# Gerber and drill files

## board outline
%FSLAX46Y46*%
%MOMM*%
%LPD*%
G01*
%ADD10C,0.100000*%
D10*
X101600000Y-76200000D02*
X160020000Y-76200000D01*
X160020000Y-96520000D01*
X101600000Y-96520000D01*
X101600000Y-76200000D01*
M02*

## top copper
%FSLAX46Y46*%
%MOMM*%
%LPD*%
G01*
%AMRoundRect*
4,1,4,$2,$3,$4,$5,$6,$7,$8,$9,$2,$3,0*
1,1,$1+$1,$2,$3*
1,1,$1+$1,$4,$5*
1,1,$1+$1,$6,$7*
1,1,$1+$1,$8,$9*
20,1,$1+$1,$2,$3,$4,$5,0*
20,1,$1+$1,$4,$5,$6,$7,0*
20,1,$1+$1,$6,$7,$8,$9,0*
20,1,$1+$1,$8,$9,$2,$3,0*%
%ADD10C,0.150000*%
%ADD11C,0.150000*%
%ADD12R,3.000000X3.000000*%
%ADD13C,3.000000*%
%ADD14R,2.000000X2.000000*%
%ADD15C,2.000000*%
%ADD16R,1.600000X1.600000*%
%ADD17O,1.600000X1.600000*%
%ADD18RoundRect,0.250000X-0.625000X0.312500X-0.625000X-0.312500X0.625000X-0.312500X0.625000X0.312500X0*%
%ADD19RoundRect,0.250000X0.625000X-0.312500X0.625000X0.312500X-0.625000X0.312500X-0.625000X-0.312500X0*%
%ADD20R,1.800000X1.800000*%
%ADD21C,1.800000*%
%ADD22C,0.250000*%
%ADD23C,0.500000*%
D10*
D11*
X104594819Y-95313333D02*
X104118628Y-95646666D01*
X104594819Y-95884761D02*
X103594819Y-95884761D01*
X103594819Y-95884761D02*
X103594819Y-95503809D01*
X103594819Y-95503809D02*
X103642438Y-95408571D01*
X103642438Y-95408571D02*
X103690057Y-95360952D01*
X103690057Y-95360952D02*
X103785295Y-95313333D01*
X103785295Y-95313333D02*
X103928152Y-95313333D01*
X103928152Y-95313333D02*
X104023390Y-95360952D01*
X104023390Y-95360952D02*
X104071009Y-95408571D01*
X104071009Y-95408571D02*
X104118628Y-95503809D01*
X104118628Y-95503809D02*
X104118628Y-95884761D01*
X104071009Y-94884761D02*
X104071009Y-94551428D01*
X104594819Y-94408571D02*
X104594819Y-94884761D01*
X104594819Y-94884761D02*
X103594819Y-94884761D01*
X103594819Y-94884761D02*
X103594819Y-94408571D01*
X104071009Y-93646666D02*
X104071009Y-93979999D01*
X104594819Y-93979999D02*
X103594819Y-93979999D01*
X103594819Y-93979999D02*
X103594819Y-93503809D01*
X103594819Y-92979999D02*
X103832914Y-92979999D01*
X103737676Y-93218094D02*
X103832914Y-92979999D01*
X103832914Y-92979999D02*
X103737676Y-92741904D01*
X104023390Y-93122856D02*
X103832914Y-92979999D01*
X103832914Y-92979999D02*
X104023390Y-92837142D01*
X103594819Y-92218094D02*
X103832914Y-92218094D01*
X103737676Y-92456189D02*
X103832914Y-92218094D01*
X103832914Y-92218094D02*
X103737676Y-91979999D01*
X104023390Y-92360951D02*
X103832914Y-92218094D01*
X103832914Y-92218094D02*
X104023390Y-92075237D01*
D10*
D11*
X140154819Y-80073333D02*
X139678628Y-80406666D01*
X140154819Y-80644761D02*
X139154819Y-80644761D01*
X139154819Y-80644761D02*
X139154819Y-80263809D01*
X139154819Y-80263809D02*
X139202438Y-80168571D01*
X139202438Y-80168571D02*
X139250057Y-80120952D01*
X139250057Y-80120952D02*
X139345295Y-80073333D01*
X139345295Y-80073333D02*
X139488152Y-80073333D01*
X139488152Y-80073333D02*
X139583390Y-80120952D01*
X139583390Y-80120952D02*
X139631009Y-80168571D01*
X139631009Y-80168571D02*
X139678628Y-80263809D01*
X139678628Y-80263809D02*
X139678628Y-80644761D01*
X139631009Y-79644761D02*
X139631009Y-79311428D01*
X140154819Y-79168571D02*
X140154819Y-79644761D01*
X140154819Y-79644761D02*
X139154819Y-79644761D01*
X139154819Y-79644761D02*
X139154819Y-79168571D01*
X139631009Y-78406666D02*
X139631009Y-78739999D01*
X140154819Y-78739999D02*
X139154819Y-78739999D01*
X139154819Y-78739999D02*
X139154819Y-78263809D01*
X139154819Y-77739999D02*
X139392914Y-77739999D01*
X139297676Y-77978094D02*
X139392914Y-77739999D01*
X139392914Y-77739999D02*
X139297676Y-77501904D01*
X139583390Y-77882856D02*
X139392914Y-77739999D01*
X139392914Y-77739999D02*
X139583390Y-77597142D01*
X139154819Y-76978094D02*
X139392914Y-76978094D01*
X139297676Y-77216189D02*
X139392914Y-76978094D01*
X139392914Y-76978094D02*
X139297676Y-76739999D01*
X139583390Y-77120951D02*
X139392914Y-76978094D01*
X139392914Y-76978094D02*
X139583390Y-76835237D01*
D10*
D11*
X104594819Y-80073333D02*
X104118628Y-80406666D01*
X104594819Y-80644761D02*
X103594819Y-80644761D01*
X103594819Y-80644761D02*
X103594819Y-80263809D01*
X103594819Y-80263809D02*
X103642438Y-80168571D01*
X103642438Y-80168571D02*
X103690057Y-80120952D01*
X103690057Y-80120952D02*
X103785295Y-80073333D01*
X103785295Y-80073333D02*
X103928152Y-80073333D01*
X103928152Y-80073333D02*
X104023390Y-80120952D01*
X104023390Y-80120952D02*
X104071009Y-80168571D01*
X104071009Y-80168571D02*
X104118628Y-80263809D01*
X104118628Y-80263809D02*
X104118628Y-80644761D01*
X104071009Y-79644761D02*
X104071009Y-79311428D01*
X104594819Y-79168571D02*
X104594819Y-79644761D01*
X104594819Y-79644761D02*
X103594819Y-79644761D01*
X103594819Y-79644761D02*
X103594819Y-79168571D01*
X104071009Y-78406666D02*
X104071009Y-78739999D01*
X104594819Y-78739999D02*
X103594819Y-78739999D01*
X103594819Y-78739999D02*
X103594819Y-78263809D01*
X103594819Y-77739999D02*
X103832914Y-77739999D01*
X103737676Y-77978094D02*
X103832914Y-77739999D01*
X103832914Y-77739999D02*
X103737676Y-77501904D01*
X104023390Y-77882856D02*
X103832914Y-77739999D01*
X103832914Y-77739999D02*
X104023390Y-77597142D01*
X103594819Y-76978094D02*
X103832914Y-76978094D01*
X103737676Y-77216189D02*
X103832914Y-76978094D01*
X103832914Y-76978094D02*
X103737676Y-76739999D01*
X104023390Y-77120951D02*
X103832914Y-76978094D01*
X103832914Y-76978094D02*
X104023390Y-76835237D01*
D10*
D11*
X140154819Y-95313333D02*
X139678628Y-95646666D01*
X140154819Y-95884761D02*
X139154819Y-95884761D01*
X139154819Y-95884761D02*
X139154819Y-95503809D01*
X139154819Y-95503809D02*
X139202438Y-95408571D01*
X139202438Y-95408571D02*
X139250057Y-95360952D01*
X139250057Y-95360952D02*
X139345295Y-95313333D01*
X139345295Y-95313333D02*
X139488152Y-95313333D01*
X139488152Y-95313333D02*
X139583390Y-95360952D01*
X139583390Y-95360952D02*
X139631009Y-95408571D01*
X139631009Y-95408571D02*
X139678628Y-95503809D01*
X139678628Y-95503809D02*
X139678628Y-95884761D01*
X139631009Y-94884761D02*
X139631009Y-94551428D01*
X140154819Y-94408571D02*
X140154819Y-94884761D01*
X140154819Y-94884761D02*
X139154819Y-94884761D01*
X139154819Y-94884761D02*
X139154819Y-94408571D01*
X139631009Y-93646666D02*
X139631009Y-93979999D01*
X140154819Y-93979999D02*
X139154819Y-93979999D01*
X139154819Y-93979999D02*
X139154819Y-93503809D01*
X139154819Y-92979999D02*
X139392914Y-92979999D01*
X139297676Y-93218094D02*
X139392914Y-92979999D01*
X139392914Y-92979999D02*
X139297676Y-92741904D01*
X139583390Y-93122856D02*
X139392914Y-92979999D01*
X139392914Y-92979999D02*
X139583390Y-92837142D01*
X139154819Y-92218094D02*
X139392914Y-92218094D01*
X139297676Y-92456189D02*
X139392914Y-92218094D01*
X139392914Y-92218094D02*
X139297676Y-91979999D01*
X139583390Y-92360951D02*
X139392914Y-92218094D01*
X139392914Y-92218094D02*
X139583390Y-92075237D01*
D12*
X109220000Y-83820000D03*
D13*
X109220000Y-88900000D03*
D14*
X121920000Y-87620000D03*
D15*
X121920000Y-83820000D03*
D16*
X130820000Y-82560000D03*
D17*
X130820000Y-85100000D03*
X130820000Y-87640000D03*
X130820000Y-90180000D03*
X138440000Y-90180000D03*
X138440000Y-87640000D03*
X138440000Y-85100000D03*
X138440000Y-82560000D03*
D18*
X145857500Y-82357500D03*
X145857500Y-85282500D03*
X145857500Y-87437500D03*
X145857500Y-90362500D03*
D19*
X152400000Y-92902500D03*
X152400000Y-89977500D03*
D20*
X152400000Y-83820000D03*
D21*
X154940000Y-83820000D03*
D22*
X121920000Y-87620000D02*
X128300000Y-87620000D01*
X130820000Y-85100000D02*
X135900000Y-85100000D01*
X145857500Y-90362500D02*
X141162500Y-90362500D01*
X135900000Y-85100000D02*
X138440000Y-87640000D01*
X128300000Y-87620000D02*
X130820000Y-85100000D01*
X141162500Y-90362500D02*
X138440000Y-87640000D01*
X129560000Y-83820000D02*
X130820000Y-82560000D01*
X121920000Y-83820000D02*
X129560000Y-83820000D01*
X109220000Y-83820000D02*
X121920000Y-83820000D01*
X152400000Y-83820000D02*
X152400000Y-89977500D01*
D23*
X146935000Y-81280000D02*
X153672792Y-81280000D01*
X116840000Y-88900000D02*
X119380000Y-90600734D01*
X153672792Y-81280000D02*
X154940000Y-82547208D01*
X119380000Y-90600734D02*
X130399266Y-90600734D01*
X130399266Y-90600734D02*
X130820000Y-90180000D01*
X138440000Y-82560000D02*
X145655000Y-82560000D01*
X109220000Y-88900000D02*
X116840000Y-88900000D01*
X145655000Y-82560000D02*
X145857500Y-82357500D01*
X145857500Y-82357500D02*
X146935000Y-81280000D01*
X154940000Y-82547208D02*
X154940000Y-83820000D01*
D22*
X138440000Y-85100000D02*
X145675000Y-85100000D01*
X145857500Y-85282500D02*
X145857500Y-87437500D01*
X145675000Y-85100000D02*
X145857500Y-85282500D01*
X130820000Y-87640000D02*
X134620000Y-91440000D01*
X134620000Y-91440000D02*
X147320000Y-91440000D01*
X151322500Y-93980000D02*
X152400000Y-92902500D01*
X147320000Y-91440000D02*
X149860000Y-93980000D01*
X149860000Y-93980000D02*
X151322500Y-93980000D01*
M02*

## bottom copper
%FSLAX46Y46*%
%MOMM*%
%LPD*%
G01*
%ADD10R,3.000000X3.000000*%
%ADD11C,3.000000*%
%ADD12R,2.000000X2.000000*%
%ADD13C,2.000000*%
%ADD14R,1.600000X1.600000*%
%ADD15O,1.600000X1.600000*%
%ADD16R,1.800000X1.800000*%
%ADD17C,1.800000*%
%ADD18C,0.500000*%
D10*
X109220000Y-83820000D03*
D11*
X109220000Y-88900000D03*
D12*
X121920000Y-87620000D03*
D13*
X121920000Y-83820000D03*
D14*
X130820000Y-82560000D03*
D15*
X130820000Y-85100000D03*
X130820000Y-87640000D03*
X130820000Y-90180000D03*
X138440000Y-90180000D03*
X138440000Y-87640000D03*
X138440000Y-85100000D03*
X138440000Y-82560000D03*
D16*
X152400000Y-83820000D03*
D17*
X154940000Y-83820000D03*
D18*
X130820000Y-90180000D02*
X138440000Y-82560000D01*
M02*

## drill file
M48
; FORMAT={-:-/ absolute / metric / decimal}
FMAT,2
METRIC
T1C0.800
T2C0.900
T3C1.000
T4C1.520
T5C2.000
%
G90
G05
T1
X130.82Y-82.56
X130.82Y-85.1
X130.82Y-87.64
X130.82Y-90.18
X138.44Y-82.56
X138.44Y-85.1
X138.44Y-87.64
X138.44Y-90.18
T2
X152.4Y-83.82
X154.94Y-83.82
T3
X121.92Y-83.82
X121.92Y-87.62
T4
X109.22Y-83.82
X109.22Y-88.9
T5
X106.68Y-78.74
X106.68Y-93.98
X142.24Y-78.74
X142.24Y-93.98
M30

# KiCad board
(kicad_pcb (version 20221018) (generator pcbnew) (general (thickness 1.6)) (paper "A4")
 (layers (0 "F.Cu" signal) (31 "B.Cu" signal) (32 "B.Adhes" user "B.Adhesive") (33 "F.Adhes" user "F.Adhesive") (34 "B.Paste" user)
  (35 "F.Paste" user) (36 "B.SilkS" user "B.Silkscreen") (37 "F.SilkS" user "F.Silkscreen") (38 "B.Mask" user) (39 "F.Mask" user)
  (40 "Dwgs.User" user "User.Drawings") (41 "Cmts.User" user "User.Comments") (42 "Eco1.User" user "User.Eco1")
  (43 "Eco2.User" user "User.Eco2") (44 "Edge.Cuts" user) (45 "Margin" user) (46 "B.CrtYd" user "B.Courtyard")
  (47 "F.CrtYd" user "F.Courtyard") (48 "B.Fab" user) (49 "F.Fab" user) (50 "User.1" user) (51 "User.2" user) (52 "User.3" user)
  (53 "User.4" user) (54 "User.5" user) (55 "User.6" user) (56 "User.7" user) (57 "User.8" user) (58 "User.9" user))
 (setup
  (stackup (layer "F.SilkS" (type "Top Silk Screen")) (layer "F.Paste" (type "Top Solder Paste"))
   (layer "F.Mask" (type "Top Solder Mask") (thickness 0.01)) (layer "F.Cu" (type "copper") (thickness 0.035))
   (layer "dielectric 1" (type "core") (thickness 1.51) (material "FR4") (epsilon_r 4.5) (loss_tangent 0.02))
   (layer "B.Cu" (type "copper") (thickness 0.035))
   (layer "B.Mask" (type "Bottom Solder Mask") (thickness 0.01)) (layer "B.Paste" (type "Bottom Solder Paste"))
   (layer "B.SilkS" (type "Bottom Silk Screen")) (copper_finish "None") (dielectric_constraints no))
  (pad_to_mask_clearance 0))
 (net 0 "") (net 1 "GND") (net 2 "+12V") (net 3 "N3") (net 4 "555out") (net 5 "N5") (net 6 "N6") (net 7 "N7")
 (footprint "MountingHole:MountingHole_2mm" (layer "F.Cu") (at 106.68 93.98)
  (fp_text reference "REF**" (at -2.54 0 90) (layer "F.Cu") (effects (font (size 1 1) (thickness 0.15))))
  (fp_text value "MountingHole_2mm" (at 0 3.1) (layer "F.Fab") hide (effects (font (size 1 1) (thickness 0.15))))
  (pad "" np_thru_hole circle (at 0 0) (size 2 2) (drill 2) (layers "*.Cu" "*.Mask")))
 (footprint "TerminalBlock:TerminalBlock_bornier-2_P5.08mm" (layer "F.Cu") (at 109.22 83.82 -90)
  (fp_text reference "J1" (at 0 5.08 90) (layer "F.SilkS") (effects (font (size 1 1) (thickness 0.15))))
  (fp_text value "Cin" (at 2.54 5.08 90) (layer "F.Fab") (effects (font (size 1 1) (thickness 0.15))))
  (pad "1" thru_hole rect (at 0 0 270) (size 3 3) (drill 1.52) (layers "*.Cu" "*.Mask") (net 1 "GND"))
  (pad "2" thru_hole circle (at 5.08 0 270) (size 3 3) (drill 1.52) (layers "*.Cu" "*.Mask") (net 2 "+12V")))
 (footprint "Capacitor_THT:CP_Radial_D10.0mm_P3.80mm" (layer "F.Cu") (at 121.92 87.62 90)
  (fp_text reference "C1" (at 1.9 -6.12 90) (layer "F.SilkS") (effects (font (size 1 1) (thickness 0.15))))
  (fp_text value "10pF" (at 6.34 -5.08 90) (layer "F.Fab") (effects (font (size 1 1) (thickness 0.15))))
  (pad "1" thru_hole rect (at 0 0 90) (size 2 2) (drill 1) (layers "*.Cu" "*.Mask") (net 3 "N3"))
  (pad "2" thru_hole circle (at 3.8 0 90) (size 2 2) (drill 1) (layers "*.Cu" "*.Mask") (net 1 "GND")))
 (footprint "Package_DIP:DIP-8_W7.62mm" (layer "F.Cu") (at 130.82 82.56)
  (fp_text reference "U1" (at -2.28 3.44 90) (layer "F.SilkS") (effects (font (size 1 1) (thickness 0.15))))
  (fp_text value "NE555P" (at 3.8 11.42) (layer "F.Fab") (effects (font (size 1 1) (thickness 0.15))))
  (pad "1" thru_hole rect (at 0 0) (size 1.6 1.6) (drill 0.8) (layers "*.Cu" "*.Mask") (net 1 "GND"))
  (pad "2" thru_hole oval (at 0 2.54) (size 1.6 1.6) (drill 0.8) (layers "*.Cu" "*.Mask") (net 3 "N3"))
  (pad "3" thru_hole oval (at 0 5.08) (size 1.6 1.6) (drill 0.8) (layers "*.Cu" "*.Mask") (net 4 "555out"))
  (pad "4" thru_hole oval (at 0 7.62) (size 1.6 1.6) (drill 0.8) (layers "*.Cu" "*.Mask") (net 2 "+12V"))
  (pad "5" thru_hole oval (at 7.62 7.62) (size 1.6 1.6) (drill 0.8) (layers "*.Cu" "*.Mask") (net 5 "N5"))
  (pad "6" thru_hole oval (at 7.62 5.08) (size 1.6 1.6) (drill 0.8) (layers "*.Cu" "*.Mask") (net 3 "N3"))
  (pad "7" thru_hole oval (at 7.62 2.54) (size 1.6 1.6) (drill 0.8) (layers "*.Cu" "*.Mask") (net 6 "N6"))
  (pad "8" thru_hole oval (at 7.62 0) (size 1.6 1.6) (drill 0.8) (layers "*.Cu" "*.Mask") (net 2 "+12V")))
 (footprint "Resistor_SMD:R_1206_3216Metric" (layer "F.Cu") (at 145.8575 83.82 -90)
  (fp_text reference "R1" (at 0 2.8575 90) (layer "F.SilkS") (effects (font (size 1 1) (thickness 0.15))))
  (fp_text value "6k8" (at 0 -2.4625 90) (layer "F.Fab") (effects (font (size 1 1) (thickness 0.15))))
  (pad "1" smd roundrect (at -1.4625 0 270) (size 1.125 1.75) (layers "F.Cu" "F.Paste" "F.Mask") (roundrect_rratio 0.222222) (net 2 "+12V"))
  (pad "2" smd roundrect (at 1.4625 0 270) (size 1.125 1.75) (layers "F.Cu" "F.Paste" "F.Mask") (roundrect_rratio 0.222222) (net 6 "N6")))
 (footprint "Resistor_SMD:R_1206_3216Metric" (layer "F.Cu") (at 145.8575 88.9 -90)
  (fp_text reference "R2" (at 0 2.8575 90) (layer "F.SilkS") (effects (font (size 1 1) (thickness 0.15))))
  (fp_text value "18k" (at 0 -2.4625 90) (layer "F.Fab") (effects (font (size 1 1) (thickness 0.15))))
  (pad "1" smd roundrect (at -1.4625 0 270) (size 1.125 1.75) (layers "F.Cu" "F.Paste" "F.Mask") (roundrect_rratio 0.222222) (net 6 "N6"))
  (pad "2" smd roundrect (at 1.4625 0 270) (size 1.125 1.75) (layers "F.Cu" "F.Paste" "F.Mask") (roundrect_rratio 0.222222) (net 3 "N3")))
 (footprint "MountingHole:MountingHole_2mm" (layer "F.Cu") (at 142.24 78.74)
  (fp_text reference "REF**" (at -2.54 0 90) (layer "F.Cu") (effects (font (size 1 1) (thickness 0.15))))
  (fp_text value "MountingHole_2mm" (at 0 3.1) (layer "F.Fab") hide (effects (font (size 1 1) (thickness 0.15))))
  (pad "" np_thru_hole circle (at 0 0) (size 2 2) (drill 2) (layers "*.Cu" "*.Mask")))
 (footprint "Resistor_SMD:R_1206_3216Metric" (layer "F.Cu") (at 152.4 91.44 90)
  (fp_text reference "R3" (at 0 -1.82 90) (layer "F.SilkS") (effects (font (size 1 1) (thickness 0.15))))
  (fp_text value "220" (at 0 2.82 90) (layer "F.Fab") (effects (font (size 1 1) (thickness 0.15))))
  (pad "1" smd roundrect (at -1.4625 0 90) (size 1.125 1.75) (layers "F.Cu" "F.Paste" "F.Mask") (roundrect_rratio 0.222222) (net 4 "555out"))
  (pad "2" smd roundrect (at 1.4625 0 90) (size 1.125 1.75) (layers "F.Cu" "F.Paste" "F.Mask") (roundrect_rratio 0.222222) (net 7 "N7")))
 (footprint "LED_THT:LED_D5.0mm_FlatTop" (layer "F.Cu") (at 152.4 83.82)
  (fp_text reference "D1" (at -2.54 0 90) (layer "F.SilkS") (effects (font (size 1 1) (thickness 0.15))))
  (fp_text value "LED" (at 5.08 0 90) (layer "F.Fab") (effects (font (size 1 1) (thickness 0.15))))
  (pad "1" thru_hole rect (at 0 0) (size 1.8 1.8) (drill 0.9) (layers "*.Cu" "*.Mask") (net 7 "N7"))
  (pad "2" thru_hole circle (at 2.54 0) (size 1.8 1.8) (drill 0.9) (layers "*.Cu" "*.Mask") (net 2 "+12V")))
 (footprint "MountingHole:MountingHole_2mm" (layer "F.Cu") (at 106.68 78.74)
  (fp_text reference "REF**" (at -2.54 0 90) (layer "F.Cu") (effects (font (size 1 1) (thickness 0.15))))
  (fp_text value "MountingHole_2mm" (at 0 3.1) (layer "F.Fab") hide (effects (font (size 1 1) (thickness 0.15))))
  (pad "" np_thru_hole circle (at 0 0) (size 2 2) (drill 2) (layers "*.Cu" "*.Mask")))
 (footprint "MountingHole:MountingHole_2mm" (layer "F.Cu") (at 142.24 93.98)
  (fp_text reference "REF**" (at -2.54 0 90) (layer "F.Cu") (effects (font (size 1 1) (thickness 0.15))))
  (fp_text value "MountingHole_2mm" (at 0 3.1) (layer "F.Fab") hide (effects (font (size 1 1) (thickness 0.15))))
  (pad "" np_thru_hole circle (at 0 0) (size 2 2) (drill 2) (layers "*.Cu" "*.Mask")))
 (gr_rect (start 101.6 76.2) (end 160.02 96.52) (stroke (width 0.1) (type default)) (fill none) (layer "Edge.Cuts"))
 (segment (start 121.92 87.62) (end 128.3 87.62) (width 0.25) (layer "F.Cu") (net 3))
 (segment (start 130.82 85.1) (end 135.9 85.1) (width 0.25) (layer "F.Cu") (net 3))
 (segment (start 145.8575 90.3625) (end 141.1625 90.3625) (width 0.25) (layer "F.Cu") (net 3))
 (segment (start 135.9 85.1) (end 138.44 87.64) (width 0.25) (layer "F.Cu") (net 3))
 (segment (start 128.3 87.62) (end 130.82 85.1) (width 0.25) (layer "F.Cu") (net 3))
 (segment (start 141.1625 90.3625) (end 138.44 87.64) (width 0.25) (layer "F.Cu") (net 3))
 (segment (start 129.56 83.82) (end 130.82 82.56) (width 0.25) (layer "F.Cu") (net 1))
 (segment (start 121.92 83.82) (end 129.56 83.82) (width 0.25) (layer "F.Cu") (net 1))
 (segment (start 109.22 83.82) (end 121.92 83.82) (width 0.25) (layer "F.Cu") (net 1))
 (segment (start 152.4 83.82) (end 152.4 89.9775) (width 0.25) (layer "F.Cu") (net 7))
 (segment (start 146.935 81.28) (end 153.672792 81.28) (width 0.5) (layer "F.Cu") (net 2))
 (segment (start 116.84 88.9) (end 119.38 90.600734) (width 0.5) (layer "F.Cu") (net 2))
 (segment (start 153.672792 81.28) (end 154.94 82.547208) (width 0.5) (layer "F.Cu") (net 2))
 (segment (start 119.38 90.600734) (end 130.399266 90.600734) (width 0.5) (layer "F.Cu") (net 2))
 (segment (start 130.399266 90.600734) (end 130.82 90.18) (width 0.5) (layer "F.Cu") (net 2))
 (segment (start 138.44 82.56) (end 145.655 82.56) (width 0.5) (layer "F.Cu") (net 2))
 (segment (start 109.22 88.9) (end 116.84 88.9) (width 0.5) (layer "F.Cu") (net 2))
 (segment (start 145.655 82.56) (end 145.8575 82.3575) (width 0.5) (layer "F.Cu") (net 2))
 (segment (start 145.8575 82.3575) (end 146.935 81.28) (width 0.5) (layer "F.Cu") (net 2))
 (segment (start 154.94 82.547208) (end 154.94 83.82) (width 0.5) (layer "F.Cu") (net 2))
 (segment (start 130.82 90.18) (end 138.44 82.56) (width 0.5) (layer "B.Cu") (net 2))
 (segment (start 138.44 85.1) (end 145.675 85.1) (width 0.25) (layer "F.Cu") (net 6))
 (segment (start 145.8575 85.2825) (end 145.8575 87.4375) (width 0.25) (layer "F.Cu") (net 6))
 (segment (start 145.675 85.1) (end 145.8575 85.2825) (width 0.25) (layer "F.Cu") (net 6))
 (segment (start 130.82 87.64) (end 134.62 91.44) (width 0.25) (layer "F.Cu") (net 4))
 (segment (start 134.62 91.44) (end 147.32 91.44) (width 0.25) (layer "F.Cu") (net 4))
 (segment (start 151.3225 93.98) (end 152.4 92.9025) (width 0.25) (layer "F.Cu") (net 4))
 (segment (start 147.32 91.44) (end 149.86 93.98) (width 0.25) (layer "F.Cu") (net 4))
 (segment (start 149.86 93.98) (end 151.3225 93.98) (width 0.25) (layer "F.Cu") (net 4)))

